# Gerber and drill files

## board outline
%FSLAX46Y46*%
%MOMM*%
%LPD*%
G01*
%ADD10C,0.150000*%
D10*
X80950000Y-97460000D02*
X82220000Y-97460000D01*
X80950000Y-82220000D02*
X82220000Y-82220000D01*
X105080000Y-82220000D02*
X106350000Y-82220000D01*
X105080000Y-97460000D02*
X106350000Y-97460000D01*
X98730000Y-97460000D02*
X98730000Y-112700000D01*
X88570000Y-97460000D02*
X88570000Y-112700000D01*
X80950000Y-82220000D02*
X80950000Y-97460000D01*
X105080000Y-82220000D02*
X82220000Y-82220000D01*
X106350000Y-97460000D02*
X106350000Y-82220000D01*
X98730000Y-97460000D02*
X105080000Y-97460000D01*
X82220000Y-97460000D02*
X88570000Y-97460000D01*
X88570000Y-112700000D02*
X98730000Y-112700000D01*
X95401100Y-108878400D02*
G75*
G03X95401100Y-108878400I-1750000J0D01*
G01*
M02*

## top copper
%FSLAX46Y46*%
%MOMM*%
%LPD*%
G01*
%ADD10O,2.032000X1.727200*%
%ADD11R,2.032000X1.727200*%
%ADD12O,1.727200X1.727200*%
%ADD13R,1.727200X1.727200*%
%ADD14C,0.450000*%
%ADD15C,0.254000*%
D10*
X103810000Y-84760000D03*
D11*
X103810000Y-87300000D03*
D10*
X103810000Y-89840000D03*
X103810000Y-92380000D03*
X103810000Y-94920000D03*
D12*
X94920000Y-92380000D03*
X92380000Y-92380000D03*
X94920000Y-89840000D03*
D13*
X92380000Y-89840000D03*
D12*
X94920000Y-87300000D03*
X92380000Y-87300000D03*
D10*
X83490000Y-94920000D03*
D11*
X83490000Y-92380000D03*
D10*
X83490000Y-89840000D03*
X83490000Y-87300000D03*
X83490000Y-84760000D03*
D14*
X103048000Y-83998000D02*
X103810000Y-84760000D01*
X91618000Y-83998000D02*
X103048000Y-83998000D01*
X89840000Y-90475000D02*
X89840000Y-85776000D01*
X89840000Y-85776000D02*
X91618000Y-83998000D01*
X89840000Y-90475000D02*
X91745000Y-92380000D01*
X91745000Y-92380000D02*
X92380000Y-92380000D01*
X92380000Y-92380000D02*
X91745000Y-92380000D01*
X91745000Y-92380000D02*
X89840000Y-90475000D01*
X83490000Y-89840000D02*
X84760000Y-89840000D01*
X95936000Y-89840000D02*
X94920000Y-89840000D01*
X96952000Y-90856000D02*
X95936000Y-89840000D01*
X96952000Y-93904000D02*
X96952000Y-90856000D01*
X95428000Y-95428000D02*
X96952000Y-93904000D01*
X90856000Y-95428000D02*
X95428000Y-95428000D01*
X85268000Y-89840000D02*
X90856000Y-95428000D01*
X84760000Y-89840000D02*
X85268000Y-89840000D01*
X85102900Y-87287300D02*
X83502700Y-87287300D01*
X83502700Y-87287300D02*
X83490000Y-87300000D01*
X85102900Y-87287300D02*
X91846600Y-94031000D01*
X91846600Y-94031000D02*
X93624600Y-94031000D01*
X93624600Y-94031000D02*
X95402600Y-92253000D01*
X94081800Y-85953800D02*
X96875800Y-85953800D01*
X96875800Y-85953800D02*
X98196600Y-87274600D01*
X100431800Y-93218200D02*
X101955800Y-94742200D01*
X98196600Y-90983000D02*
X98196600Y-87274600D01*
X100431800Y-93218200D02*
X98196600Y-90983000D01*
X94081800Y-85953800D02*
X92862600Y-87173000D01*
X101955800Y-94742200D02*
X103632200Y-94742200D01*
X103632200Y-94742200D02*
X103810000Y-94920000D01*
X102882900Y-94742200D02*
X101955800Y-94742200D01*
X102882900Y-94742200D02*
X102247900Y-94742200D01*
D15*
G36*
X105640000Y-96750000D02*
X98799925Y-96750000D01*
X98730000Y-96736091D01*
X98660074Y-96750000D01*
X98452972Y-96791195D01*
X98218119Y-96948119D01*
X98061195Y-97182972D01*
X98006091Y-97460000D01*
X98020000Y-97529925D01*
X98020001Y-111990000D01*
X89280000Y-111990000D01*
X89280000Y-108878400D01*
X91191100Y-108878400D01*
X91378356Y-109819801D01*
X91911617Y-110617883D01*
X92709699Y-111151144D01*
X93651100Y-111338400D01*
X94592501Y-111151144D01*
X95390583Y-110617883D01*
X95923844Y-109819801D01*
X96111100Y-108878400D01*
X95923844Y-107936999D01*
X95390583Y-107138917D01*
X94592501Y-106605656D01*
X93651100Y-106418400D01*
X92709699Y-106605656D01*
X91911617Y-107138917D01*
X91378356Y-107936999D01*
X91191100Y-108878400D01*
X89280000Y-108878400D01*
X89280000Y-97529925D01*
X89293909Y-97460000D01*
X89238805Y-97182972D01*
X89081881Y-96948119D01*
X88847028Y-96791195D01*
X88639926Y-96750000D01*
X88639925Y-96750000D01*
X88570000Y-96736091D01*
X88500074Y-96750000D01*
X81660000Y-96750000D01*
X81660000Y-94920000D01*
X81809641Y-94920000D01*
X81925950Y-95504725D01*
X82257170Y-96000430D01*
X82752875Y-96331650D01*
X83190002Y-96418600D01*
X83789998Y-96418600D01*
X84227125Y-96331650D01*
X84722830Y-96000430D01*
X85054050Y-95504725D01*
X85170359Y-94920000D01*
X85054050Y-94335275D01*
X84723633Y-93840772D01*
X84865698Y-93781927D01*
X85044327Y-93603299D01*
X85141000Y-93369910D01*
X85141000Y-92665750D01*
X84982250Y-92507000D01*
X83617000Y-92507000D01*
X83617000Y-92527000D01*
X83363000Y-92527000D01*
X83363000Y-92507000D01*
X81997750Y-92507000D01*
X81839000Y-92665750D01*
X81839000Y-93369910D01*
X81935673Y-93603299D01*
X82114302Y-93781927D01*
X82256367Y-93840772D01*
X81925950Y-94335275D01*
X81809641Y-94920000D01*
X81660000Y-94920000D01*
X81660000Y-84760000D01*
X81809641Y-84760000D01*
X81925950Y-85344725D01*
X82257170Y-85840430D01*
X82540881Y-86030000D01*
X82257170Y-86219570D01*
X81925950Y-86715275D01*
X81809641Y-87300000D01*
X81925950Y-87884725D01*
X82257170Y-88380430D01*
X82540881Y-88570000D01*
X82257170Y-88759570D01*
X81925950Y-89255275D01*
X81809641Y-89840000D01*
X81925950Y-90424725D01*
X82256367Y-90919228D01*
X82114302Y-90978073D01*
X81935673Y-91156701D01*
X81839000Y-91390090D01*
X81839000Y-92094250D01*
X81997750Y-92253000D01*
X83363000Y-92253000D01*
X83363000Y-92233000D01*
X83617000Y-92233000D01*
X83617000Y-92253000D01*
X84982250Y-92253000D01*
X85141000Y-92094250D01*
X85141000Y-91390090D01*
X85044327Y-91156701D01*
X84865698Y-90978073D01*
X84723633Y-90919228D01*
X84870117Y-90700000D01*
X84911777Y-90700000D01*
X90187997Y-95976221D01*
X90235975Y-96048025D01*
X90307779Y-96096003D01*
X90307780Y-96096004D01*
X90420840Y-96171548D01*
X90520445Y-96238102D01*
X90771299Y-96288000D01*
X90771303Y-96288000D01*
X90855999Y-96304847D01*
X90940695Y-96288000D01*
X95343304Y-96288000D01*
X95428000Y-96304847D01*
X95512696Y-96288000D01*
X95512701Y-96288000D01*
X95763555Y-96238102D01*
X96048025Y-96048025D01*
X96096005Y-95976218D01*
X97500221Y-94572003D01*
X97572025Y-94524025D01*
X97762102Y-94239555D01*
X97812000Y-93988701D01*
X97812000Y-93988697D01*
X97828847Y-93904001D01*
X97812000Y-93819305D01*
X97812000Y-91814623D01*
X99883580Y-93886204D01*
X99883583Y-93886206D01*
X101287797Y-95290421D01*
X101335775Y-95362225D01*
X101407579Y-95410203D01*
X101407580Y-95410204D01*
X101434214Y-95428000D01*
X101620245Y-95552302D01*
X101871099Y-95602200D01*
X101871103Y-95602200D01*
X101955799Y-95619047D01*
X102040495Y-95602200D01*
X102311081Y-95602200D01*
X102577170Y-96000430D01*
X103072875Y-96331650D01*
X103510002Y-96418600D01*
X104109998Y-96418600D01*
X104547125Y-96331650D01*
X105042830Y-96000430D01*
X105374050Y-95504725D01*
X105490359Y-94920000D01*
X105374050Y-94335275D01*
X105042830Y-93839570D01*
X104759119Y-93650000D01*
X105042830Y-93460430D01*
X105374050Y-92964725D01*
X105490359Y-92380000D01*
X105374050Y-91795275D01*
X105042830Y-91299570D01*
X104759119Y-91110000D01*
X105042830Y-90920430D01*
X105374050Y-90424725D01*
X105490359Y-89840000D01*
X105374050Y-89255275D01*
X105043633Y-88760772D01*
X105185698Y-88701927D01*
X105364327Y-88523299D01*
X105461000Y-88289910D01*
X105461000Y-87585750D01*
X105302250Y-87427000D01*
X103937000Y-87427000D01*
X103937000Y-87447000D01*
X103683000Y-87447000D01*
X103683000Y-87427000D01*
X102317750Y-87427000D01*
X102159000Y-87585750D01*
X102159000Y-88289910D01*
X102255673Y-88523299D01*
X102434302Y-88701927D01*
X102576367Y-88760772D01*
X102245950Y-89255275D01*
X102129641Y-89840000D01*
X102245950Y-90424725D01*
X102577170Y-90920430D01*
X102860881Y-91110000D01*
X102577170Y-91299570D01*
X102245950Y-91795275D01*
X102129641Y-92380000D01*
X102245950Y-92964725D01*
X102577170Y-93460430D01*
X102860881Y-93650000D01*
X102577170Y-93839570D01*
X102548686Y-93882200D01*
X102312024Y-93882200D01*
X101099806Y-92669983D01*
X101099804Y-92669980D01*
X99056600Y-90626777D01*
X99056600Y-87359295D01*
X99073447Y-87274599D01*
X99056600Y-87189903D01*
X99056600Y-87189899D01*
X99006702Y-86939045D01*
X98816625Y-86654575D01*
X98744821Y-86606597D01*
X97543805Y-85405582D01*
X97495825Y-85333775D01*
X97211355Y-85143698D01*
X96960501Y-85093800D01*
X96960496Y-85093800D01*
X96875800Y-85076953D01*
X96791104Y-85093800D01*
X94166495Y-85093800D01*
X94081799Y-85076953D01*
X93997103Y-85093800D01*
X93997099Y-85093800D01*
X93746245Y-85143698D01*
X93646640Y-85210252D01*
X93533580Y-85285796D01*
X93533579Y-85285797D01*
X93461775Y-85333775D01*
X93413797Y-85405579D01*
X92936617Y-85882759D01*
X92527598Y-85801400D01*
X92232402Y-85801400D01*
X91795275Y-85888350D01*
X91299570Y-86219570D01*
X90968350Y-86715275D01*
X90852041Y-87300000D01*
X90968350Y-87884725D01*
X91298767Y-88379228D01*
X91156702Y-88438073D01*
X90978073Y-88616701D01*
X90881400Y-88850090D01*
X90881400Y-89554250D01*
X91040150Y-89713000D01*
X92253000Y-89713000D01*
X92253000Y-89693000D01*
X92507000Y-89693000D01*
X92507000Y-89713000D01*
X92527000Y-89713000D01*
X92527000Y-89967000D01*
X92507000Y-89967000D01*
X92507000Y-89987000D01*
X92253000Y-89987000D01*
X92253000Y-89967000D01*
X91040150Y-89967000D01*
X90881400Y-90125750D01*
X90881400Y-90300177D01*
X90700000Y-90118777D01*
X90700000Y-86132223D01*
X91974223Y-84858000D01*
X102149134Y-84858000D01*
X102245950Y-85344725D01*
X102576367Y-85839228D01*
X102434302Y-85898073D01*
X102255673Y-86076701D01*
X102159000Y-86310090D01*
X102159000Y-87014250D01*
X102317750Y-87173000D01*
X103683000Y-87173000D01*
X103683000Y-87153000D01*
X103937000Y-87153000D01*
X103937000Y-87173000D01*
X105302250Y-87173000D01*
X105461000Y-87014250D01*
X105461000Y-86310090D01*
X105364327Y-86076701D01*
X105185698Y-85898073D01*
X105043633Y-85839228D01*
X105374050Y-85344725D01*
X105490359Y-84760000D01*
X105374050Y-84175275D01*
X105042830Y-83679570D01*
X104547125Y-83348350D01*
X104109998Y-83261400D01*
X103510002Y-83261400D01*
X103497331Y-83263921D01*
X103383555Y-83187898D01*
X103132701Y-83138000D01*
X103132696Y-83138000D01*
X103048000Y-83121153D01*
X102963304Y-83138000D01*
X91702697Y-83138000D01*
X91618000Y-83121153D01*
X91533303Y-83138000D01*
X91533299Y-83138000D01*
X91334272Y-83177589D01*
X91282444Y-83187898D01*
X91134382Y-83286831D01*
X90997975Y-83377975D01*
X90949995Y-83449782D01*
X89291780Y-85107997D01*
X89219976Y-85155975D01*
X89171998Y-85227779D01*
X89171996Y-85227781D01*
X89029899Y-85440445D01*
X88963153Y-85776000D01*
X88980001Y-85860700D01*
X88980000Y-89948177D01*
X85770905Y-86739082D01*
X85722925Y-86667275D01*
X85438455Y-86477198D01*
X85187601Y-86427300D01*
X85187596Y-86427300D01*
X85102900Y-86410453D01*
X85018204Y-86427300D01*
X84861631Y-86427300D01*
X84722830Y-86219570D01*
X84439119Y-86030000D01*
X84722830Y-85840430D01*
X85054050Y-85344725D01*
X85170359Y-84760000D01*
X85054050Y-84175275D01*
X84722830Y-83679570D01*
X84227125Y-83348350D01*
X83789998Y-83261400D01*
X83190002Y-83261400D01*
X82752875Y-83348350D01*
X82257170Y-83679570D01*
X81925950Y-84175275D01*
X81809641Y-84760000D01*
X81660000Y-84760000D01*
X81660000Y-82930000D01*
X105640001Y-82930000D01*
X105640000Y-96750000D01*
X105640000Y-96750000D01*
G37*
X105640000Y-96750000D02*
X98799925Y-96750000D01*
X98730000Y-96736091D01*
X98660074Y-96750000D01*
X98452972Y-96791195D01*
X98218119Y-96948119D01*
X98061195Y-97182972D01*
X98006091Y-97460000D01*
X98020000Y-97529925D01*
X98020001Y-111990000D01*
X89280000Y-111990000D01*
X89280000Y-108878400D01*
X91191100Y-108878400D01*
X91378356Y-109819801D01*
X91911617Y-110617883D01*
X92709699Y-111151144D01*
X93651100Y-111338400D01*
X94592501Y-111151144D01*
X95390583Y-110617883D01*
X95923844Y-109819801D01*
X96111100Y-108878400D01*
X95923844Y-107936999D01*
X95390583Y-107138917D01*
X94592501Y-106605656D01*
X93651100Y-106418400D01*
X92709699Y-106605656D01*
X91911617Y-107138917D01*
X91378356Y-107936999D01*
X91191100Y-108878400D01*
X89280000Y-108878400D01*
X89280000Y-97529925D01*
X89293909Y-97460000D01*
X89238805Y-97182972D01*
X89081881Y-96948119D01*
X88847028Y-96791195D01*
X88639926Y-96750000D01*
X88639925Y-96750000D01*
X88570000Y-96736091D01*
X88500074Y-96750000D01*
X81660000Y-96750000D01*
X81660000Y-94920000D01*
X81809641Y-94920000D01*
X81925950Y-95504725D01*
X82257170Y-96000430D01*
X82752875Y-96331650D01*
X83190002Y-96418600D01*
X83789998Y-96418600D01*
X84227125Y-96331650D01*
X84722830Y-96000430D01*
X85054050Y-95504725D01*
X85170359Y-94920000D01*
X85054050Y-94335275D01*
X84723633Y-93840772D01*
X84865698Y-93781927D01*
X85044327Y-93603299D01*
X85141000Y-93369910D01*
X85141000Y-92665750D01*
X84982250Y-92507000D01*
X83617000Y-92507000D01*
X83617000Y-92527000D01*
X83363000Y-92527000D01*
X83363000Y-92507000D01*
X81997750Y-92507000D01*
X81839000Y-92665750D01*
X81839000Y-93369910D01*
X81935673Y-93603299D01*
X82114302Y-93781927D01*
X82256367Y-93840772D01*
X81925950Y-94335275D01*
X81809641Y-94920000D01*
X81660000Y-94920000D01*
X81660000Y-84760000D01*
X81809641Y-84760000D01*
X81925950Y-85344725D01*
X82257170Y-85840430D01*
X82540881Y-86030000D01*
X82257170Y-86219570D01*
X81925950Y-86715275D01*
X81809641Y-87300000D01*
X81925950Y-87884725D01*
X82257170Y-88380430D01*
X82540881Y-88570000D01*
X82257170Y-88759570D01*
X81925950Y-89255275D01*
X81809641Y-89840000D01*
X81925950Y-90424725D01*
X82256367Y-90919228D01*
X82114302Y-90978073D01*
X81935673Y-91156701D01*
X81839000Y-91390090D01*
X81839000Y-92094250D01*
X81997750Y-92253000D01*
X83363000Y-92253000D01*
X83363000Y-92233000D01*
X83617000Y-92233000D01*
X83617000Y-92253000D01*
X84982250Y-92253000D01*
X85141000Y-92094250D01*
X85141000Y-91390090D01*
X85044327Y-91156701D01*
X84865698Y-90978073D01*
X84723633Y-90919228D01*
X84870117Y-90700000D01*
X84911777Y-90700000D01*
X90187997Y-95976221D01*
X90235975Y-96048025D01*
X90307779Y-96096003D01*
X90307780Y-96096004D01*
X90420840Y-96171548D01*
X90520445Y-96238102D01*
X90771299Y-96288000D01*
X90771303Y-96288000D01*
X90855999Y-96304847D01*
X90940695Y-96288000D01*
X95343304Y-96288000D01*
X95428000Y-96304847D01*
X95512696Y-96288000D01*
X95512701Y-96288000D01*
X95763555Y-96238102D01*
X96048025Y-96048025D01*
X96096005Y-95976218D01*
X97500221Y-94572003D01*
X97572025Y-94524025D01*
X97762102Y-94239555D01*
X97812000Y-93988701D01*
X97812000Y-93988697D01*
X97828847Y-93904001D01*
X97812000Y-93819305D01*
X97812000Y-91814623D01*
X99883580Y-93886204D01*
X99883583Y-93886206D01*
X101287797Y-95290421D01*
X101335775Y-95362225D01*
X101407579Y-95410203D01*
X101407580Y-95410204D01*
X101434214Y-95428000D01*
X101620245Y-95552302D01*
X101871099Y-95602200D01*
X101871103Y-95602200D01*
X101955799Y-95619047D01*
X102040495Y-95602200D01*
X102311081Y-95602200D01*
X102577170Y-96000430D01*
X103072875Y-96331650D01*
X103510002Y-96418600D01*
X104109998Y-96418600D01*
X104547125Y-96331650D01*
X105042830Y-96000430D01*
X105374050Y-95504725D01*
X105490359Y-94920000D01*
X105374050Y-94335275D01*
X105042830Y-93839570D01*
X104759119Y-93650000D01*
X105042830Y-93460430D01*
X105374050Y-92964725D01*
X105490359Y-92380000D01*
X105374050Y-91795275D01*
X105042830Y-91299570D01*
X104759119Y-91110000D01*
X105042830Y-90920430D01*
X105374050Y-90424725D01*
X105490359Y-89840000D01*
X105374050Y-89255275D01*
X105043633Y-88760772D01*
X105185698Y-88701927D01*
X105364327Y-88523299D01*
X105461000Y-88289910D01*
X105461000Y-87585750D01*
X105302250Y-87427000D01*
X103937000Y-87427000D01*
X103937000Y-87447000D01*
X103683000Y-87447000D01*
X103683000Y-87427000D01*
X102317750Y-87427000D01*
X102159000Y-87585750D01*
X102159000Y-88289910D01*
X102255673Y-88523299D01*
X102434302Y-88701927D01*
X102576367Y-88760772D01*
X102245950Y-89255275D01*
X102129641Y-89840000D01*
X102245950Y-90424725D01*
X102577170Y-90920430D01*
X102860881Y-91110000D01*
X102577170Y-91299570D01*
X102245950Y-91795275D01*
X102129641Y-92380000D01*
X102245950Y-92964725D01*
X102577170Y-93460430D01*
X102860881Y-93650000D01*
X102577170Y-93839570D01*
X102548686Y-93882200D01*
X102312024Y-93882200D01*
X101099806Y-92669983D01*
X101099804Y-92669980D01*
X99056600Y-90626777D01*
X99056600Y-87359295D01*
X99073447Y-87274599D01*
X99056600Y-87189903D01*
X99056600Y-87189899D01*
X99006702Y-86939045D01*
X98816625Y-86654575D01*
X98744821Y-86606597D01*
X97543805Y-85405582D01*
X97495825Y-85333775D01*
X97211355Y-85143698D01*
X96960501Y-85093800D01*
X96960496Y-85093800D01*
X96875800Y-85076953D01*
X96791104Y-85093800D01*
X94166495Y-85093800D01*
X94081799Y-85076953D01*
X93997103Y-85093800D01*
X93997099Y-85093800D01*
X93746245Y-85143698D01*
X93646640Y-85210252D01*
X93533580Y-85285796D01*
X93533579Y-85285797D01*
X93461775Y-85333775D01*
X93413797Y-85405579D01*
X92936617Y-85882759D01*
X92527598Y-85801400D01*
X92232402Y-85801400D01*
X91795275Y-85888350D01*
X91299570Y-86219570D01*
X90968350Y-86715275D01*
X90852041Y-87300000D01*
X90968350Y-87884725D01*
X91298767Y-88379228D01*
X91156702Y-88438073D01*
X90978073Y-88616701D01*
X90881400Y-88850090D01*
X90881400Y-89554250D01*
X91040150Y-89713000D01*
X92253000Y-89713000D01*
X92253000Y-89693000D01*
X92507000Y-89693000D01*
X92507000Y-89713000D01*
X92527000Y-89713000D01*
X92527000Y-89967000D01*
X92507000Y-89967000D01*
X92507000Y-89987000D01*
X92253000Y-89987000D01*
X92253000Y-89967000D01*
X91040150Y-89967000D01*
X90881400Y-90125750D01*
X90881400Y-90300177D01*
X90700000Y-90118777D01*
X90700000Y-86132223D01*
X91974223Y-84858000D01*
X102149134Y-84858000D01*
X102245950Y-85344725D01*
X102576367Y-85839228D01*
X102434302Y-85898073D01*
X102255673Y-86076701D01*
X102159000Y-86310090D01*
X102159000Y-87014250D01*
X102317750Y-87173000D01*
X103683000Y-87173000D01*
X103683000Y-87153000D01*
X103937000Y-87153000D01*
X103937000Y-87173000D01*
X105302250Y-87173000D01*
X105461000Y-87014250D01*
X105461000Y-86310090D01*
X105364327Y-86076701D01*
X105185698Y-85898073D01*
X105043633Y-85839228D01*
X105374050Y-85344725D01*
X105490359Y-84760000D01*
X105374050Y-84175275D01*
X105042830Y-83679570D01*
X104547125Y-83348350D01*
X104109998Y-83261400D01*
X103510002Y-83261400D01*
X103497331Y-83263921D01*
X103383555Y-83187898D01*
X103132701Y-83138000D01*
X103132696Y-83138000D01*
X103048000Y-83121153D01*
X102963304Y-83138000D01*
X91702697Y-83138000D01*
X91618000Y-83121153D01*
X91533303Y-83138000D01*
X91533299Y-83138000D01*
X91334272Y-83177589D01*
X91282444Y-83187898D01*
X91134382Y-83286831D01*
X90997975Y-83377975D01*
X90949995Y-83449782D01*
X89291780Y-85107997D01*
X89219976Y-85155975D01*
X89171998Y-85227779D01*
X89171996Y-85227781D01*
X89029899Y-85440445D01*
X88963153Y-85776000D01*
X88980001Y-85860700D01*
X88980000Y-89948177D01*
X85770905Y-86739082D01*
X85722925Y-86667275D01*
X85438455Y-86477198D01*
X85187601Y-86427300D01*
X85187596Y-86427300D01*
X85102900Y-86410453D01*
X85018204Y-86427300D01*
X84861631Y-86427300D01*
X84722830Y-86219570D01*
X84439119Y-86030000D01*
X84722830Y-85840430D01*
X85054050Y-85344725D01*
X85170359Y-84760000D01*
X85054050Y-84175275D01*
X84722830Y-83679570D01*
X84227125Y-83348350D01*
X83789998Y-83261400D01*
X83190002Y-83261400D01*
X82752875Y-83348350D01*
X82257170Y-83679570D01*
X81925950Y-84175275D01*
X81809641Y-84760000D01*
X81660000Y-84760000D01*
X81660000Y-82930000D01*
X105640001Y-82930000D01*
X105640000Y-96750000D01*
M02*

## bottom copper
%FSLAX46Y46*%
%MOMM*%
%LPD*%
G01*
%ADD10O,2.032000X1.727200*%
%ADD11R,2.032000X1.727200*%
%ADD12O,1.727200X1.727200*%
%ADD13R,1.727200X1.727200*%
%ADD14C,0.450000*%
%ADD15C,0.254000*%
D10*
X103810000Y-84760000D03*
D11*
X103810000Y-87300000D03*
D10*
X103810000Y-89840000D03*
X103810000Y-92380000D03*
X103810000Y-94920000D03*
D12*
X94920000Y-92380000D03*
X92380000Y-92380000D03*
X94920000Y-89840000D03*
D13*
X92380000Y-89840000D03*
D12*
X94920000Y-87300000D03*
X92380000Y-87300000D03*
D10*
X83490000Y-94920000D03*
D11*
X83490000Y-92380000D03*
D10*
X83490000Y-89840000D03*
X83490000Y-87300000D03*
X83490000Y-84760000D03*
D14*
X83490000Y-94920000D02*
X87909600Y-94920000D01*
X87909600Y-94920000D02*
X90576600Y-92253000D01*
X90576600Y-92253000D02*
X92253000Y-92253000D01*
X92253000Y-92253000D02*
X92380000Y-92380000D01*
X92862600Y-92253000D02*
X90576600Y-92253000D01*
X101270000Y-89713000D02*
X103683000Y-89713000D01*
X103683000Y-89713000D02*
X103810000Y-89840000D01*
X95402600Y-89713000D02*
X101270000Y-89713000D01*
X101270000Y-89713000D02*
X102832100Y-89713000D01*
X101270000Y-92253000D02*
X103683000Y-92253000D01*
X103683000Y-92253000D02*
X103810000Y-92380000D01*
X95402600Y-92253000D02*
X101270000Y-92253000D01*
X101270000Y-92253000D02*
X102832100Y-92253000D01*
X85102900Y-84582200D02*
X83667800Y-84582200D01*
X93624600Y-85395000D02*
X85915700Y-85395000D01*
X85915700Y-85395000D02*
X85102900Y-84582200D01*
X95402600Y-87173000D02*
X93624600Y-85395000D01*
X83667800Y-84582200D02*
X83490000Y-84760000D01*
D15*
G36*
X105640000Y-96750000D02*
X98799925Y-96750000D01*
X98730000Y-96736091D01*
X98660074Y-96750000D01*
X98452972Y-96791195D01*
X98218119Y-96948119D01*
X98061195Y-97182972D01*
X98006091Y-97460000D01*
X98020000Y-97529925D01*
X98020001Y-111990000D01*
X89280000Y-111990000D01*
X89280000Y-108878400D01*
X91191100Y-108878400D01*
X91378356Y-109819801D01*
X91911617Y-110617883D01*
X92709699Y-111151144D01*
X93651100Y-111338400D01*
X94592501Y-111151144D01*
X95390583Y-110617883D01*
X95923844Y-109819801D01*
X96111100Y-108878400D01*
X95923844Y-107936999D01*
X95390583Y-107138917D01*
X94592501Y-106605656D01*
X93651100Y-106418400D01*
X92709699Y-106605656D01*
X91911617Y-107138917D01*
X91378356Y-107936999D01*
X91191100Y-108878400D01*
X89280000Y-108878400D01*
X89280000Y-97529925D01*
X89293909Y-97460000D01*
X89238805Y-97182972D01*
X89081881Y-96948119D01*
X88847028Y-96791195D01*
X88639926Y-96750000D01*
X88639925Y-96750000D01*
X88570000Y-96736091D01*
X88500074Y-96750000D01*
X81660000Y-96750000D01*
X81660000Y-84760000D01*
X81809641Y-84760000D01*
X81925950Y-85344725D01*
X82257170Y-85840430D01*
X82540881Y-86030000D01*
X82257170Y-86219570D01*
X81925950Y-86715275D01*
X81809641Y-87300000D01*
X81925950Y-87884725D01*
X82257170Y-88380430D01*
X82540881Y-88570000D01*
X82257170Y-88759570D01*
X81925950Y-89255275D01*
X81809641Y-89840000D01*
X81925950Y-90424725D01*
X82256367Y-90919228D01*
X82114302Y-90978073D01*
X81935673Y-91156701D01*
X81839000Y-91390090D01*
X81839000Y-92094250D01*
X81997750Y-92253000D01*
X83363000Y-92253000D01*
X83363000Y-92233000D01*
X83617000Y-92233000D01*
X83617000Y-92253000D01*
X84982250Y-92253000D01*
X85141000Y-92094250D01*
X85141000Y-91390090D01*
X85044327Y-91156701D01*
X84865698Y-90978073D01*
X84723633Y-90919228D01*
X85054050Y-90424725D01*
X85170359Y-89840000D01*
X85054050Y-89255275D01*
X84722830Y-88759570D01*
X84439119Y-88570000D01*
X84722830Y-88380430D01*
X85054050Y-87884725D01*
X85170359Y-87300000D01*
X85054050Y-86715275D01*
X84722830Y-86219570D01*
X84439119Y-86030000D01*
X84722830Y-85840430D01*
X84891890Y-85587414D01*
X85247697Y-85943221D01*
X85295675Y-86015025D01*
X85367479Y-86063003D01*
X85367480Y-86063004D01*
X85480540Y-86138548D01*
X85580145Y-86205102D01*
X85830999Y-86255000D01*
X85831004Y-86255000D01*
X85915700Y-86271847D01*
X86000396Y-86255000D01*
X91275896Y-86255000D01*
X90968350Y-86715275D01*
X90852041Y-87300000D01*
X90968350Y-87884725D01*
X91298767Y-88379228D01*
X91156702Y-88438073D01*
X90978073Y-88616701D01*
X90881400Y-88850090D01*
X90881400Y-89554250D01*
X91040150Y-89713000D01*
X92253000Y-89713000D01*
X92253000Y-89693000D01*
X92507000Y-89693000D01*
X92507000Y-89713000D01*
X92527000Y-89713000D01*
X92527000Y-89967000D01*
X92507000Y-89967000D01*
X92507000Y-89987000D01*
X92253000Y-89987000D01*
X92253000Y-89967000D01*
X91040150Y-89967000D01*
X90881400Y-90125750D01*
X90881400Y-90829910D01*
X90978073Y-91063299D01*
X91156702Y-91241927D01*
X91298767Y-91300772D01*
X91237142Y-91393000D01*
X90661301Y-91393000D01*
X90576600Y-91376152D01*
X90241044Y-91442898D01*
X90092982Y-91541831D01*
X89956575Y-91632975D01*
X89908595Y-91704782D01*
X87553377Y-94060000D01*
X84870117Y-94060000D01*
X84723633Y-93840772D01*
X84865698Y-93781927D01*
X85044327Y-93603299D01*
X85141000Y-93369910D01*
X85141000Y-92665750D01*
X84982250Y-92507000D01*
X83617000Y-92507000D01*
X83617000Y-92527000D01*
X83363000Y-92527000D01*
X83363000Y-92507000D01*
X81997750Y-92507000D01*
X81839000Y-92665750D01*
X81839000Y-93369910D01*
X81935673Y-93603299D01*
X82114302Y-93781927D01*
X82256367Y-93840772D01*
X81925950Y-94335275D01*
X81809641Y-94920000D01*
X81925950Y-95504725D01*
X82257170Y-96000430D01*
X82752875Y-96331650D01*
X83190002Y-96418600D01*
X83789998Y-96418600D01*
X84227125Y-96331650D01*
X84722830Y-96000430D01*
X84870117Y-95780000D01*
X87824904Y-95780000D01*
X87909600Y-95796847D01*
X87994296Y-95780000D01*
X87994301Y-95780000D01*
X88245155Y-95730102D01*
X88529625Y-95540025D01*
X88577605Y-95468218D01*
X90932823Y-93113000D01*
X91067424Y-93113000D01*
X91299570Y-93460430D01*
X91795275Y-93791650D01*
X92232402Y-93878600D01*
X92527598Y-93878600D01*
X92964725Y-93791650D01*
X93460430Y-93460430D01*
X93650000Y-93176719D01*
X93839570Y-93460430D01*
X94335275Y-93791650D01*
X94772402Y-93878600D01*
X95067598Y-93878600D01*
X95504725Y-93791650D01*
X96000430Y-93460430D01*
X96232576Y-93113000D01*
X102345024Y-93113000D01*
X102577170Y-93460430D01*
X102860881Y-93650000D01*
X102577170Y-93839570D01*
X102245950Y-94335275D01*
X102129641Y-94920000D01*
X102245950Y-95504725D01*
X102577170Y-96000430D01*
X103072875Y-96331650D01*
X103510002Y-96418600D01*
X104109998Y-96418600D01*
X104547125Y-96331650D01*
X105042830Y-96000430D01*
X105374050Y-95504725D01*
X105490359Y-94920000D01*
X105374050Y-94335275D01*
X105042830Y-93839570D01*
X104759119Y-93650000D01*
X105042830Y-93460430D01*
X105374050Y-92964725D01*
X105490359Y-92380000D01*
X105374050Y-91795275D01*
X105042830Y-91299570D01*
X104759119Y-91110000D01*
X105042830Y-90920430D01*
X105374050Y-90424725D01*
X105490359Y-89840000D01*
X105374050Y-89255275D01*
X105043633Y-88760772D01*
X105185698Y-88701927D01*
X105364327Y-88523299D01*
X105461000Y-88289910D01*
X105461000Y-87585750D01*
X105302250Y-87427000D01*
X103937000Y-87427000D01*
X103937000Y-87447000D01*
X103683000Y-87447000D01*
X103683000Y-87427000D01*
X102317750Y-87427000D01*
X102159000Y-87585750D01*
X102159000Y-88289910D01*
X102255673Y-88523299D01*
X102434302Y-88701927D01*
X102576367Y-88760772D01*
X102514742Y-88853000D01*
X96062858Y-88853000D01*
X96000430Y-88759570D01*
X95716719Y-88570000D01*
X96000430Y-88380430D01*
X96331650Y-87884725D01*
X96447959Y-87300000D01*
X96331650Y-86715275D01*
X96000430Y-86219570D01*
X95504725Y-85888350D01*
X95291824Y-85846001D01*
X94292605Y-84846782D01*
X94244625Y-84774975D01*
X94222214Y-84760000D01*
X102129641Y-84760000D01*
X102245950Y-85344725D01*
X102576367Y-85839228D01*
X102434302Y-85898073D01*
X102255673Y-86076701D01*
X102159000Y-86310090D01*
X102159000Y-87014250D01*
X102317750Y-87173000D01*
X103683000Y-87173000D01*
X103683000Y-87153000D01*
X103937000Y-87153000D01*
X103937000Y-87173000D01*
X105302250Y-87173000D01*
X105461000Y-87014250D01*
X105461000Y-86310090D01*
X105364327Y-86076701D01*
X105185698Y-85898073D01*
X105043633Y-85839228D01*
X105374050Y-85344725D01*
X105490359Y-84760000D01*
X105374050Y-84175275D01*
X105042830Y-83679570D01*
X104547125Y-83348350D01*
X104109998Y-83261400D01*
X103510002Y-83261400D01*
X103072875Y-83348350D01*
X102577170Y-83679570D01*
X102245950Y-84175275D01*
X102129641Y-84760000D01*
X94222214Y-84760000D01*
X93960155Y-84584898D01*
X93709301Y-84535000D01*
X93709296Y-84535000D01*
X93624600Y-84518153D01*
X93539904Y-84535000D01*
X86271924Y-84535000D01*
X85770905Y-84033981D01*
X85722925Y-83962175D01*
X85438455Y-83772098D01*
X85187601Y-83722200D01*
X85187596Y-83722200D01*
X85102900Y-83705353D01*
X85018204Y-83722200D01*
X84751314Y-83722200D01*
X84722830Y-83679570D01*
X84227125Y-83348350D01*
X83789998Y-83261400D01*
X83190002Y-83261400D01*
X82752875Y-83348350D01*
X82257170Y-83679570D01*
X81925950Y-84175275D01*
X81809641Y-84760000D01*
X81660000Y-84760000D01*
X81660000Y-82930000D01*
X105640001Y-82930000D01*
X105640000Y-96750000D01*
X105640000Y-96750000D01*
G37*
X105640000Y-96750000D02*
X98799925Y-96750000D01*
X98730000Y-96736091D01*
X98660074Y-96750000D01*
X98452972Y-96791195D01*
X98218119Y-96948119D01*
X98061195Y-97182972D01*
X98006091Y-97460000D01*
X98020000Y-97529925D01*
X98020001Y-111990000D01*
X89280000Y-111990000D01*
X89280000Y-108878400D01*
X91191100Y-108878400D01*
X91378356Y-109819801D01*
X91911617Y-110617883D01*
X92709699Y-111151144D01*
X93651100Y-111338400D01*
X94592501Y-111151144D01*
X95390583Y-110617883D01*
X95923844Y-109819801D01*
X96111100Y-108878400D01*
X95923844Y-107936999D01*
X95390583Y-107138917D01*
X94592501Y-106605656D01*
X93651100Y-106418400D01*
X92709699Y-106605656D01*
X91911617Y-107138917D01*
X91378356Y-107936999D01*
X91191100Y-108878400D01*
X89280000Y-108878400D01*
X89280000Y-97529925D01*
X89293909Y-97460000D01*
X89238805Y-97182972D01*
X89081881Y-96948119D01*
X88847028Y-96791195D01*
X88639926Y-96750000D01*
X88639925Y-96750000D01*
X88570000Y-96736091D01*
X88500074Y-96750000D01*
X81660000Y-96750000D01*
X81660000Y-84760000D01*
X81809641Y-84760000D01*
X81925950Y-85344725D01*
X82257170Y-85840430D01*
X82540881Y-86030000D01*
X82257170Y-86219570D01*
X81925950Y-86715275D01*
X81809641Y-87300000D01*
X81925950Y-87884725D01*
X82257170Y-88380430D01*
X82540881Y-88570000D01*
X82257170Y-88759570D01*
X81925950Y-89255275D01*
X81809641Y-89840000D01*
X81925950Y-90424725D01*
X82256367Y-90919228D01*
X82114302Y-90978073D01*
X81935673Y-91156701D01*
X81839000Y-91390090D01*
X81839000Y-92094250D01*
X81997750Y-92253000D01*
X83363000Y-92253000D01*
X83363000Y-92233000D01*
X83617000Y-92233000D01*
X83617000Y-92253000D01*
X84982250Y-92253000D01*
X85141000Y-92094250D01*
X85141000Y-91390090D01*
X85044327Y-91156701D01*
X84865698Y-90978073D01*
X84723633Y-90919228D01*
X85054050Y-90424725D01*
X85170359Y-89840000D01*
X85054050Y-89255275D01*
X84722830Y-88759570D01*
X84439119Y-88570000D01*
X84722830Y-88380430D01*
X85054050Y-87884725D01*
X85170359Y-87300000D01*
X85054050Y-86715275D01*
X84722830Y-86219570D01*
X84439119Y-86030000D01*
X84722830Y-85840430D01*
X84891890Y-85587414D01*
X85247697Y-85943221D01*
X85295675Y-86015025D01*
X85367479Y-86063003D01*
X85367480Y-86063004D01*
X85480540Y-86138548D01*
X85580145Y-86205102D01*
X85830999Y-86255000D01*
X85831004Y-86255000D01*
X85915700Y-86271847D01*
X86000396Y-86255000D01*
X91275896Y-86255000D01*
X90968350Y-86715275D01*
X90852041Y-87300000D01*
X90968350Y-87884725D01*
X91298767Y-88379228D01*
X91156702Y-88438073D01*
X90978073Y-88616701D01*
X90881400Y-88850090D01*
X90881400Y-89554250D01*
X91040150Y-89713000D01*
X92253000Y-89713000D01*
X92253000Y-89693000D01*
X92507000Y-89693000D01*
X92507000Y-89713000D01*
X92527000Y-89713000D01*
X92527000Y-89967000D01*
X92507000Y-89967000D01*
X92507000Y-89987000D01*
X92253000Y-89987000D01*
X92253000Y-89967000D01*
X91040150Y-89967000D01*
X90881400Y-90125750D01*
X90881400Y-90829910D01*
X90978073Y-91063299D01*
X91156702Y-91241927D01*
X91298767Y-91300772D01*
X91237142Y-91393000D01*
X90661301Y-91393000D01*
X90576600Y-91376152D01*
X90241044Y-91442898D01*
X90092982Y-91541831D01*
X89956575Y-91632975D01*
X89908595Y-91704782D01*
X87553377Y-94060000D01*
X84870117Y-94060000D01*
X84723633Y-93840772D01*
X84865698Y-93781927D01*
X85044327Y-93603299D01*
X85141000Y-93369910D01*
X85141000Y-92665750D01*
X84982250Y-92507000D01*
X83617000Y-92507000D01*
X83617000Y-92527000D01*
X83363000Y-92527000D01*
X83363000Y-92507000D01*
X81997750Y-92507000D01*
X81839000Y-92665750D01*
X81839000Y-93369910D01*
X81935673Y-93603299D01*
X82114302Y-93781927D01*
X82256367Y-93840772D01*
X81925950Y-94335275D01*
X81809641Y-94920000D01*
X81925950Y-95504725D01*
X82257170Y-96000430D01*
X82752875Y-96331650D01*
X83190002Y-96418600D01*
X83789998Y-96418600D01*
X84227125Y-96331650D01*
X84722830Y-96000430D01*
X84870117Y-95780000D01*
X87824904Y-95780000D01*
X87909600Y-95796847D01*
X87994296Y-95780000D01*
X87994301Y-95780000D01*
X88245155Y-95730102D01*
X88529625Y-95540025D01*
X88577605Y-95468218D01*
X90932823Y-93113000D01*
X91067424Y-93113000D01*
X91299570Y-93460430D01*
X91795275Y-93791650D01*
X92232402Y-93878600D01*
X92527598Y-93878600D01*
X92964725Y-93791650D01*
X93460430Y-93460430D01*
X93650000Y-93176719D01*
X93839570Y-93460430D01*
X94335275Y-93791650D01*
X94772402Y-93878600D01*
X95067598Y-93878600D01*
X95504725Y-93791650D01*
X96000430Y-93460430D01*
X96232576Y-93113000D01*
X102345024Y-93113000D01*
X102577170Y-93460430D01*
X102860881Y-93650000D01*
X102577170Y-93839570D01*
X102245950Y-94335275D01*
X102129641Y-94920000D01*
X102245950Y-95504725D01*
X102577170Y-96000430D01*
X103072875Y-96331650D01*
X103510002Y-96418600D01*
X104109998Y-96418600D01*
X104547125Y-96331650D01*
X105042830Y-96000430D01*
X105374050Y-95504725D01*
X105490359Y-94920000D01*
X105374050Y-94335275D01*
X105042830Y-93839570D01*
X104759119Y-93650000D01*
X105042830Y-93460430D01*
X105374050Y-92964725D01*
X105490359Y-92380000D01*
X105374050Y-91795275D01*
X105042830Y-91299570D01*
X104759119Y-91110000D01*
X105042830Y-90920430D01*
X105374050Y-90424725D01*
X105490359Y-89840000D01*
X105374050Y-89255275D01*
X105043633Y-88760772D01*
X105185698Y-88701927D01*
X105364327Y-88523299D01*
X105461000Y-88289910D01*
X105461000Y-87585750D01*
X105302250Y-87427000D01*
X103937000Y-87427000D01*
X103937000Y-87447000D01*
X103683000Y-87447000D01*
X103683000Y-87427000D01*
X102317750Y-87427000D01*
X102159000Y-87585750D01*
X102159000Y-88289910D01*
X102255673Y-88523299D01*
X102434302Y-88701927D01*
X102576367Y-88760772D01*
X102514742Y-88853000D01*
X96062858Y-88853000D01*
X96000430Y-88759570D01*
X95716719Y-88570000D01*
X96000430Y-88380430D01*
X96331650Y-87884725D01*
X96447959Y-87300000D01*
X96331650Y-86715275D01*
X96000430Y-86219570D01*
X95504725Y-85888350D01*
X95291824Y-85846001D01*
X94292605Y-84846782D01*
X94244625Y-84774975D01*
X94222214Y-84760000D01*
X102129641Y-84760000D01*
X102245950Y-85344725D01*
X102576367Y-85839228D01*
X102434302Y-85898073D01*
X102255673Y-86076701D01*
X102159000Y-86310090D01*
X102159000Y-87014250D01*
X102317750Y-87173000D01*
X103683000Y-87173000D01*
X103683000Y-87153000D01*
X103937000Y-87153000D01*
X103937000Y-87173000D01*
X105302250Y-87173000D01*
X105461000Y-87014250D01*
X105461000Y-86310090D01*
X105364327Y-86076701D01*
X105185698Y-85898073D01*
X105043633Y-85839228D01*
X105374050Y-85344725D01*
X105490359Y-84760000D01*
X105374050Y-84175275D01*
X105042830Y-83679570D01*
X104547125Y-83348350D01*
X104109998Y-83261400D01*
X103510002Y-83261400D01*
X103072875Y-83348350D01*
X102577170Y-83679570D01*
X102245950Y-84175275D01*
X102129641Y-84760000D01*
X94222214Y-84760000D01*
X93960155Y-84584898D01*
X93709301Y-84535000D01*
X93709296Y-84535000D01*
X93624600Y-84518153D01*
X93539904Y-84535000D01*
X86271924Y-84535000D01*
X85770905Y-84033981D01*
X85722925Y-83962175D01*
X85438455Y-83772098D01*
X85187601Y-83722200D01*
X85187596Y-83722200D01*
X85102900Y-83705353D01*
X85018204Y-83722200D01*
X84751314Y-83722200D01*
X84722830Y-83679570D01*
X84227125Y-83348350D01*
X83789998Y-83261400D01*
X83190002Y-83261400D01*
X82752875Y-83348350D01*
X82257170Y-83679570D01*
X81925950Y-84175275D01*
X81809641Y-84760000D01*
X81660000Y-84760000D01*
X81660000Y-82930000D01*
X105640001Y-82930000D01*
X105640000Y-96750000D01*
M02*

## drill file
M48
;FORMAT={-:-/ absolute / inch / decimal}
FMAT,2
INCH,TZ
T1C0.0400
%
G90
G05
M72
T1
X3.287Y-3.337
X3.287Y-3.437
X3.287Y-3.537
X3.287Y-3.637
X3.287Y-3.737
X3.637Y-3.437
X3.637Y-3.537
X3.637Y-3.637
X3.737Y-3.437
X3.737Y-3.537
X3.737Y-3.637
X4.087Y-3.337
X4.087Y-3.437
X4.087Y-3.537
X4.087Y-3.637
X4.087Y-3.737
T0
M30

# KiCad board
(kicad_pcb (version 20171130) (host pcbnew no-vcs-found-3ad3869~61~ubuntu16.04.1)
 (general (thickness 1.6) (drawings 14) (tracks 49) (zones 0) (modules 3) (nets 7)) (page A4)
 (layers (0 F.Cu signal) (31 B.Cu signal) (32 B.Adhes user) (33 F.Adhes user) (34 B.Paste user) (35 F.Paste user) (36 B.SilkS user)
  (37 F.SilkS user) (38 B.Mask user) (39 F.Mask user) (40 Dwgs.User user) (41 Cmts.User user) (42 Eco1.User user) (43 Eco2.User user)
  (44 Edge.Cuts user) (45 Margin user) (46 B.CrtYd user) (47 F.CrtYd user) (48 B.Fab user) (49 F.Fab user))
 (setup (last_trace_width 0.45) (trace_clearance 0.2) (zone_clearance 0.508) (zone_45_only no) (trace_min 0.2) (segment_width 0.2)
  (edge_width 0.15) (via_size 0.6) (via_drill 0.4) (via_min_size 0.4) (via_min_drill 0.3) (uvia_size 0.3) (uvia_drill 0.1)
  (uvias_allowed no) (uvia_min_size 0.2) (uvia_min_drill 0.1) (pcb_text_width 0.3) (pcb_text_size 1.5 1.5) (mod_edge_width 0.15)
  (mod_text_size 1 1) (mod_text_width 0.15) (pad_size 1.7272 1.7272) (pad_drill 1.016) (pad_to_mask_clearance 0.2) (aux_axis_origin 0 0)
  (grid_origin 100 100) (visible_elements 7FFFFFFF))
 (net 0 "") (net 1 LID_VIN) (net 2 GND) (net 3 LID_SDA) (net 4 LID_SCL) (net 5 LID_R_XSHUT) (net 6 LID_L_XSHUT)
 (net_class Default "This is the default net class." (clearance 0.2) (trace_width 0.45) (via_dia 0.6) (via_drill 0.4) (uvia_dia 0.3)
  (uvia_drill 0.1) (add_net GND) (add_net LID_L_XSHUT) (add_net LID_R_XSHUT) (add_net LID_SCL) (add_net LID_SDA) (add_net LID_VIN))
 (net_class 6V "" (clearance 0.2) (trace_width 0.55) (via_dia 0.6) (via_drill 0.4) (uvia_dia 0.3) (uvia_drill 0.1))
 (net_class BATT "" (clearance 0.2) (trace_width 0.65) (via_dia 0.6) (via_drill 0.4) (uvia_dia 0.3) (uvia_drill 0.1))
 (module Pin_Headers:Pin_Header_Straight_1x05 (layer F.Cu) (at 103.81 84.76)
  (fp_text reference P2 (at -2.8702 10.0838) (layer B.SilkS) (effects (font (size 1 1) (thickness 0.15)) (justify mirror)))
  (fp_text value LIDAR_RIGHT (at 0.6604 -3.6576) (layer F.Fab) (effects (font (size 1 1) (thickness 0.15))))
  (pad 1 thru_hole oval (at 0 0) (size 2.032 1.7272) (drill 1.016) (layers *.Cu *.Mask F.SilkS) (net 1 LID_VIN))
  (pad 2 thru_hole rect (at 0 2.54) (size 2.032 1.7272) (drill 1.016) (layers *.Cu *.Mask F.SilkS) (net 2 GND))
  (pad 3 thru_hole oval (at 0 5.08) (size 2.032 1.7272) (drill 1.016) (layers *.Cu *.Mask F.SilkS) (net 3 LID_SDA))
  (pad 4 thru_hole oval (at 0 7.62) (size 2.032 1.7272) (drill 1.016) (layers *.Cu *.Mask F.SilkS) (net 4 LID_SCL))
  (pad 5 thru_hole oval (at 0 10.16) (size 2.032 1.7272) (drill 1.016) (layers *.Cu *.Mask F.SilkS) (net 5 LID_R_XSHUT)))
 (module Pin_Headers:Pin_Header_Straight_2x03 (layer F.Cu) (at 94.92 92.38 180)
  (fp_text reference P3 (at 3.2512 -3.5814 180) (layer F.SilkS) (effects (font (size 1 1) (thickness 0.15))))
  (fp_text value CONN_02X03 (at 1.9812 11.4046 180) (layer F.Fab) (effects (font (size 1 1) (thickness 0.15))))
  (pad 1 thru_hole oval (at 0 0 180) (size 1.7272 1.7272) (drill 1.016) (layers *.Cu *.Mask F.SilkS) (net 4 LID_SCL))
  (pad 2 thru_hole oval (at 2.54 0 180) (size 1.7272 1.7272) (drill 1.016) (layers *.Cu *.Mask F.SilkS) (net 1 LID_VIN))
  (pad 3 thru_hole oval (at 0 2.54 180) (size 1.7272 1.7272) (drill 1.016) (layers *.Cu *.Mask F.SilkS) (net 3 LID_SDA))
  (pad 4 thru_hole rect (at 2.54 2.54 180) (size 1.7272 1.7272) (drill 1.016) (layers *.Cu *.Mask F.SilkS) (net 2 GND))
  (pad 5 thru_hole oval (at 0 5.08 180) (size 1.7272 1.7272) (drill 1.016) (layers *.Cu *.Mask F.SilkS) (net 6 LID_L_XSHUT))
  (pad 6 thru_hole oval (at 2.54 5.08 180) (size 1.7272 1.7272) (drill 1.016) (layers *.Cu *.Mask F.SilkS) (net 5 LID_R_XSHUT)))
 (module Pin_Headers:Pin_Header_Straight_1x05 (layer F.Cu) (at 83.49 94.92 180)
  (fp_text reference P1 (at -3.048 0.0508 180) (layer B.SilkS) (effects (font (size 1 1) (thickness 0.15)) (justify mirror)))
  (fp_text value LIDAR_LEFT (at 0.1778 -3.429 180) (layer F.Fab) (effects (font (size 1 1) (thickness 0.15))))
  (pad 1 thru_hole oval (at 0 0 180) (size 2.032 1.7272) (drill 1.016) (layers *.Cu *.Mask F.SilkS) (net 1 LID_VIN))
  (pad 2 thru_hole rect (at 0 2.54 180) (size 2.032 1.7272) (drill 1.016) (layers *.Cu *.Mask F.SilkS) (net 2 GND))
  (pad 3 thru_hole oval (at 0 5.08 180) (size 2.032 1.7272) (drill 1.016) (layers *.Cu *.Mask F.SilkS) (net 3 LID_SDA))
  (pad 4 thru_hole oval (at 0 7.62 180) (size 2.032 1.7272) (drill 1.016) (layers *.Cu *.Mask F.SilkS) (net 4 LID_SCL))
  (pad 5 thru_hole oval (at 0 10.16 180) (size 2.032 1.7272) (drill 1.016) (layers *.Cu *.Mask F.SilkS) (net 6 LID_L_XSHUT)))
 (gr_line (start 80.95 97.46) (end 82.22 97.46) (angle 90) (layer Edge.Cuts) (width 0.15))
 (gr_line (start 80.95 82.22) (end 82.22 82.22) (angle 90) (layer Edge.Cuts) (width 0.15))
 (gr_line (start 105.08 82.22) (end 106.35 82.22) (angle 90) (layer Edge.Cuts) (width 0.15))
 (gr_line (start 105.08 97.46) (end 106.35 97.46) (angle 90) (layer Edge.Cuts) (width 0.15))
 (gr_line (start 98.73 97.46) (end 98.73 112.7) (angle 90) (layer Edge.Cuts) (width 0.15))
 (gr_line (start 88.57 97.46) (end 88.57 112.7) (angle 90) (layer Edge.Cuts) (width 0.15))
 (gr_line (start 80.95 82.22) (end 80.95 97.46) (angle 90) (layer Edge.Cuts) (width 0.15))
 (gr_line (start 105.08 82.22) (end 82.22 82.22) (angle 90) (layer Edge.Cuts) (width 0.15))
 (gr_line (start 106.35 97.46) (end 106.35 82.22) (angle 90) (layer Edge.Cuts) (width 0.15))
 (gr_line (start 98.73 97.46) (end 105.08 97.46) (angle 90) (layer Edge.Cuts) (width 0.15))
 (gr_line (start 82.22 97.46) (end 88.57 97.46) (angle 90) (layer Edge.Cuts) (width 0.15))
 (gr_line (start 88.57 112.7) (end 98.73 112.7) (angle 90) (layer Edge.Cuts) (width 0.15))
 (gr_circle (center 93.6511 108.8784) (end 95.4011 108.8784) (layer Edge.Cuts) (width 0.15))
 (segment (start 103.048 83.998) (end 103.81 84.76) (width 0.45) (layer F.Cu) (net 1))
 (segment (start 91.618 83.998) (end 103.048 83.998) (width 0.45) (layer F.Cu) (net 1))
 (segment (start 89.84 90.475) (end 89.84 85.776) (width 0.45) (layer F.Cu) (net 1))
 (segment (start 89.84 85.776) (end 91.618 83.998) (width 0.45) (layer F.Cu) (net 1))
 (segment (start 83.49 94.92) (end 87.9096 94.92) (width 0.45) (layer B.Cu) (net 1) (status 400000))
 (segment (start 87.9096 94.92) (end 90.5766 92.253) (width 0.45) (layer B.Cu) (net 1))
 (segment (start 90.5766 92.253) (end 92.253 92.253) (width 0.45) (layer B.Cu) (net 1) (status 800000))
 (segment (start 92.253 92.253) (end 92.38 92.38) (width 0.45) (layer B.Cu) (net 1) (status C00000))
 (segment (start 89.84 90.475) (end 91.745 92.38) (width 0.45) (layer F.Cu) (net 1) (status 800000))
 (segment (start 91.745 92.38) (end 92.38 92.38) (width 0.45) (layer F.Cu) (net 1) (status C00000))
 (segment (start 92.38 92.38) (end 91.745 92.38) (width 0.45) (layer F.Cu) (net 1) (status C00000))
 (segment (start 91.745 92.38) (end 89.84 90.475) (width 0.45) (layer F.Cu) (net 1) (status 400000))
 (segment (start 92.8626 92.253) (end 90.5766 92.253) (width 0.45) (layer B.Cu) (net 1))
 (segment (start 101.27 89.713) (end 103.683 89.713) (width 0.45) (layer B.Cu) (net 3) (status 800000))
 (segment (start 103.683 89.713) (end 103.81 89.84) (width 0.45) (layer B.Cu) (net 3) (status C00000))
 (segment (start 83.49 89.84) (end 84.76 89.84) (width 0.45) (layer F.Cu) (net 3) (status 400000))
 (segment (start 95.936 89.84) (end 94.92 89.84) (width 0.45) (layer F.Cu) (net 3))
 (segment (start 96.952 90.856) (end 95.936 89.84) (width 0.45) (layer F.Cu) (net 3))
 (segment (start 96.952 93.904) (end 96.952 90.856) (width 0.45) (layer F.Cu) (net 3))
 (segment (start 95.428 95.428) (end 96.952 93.904) (width 0.45) (layer F.Cu) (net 3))
 (segment (start 90.856 95.428) (end 95.428 95.428) (width 0.45) (layer F.Cu) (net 3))
 (segment (start 85.268 89.84) (end 90.856 95.428) (width 0.45) (layer F.Cu) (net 3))
 (segment (start 84.76 89.84) (end 85.268 89.84) (width 0.45) (layer F.Cu) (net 3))
 (segment (start 95.4026 89.713) (end 101.27 89.713) (width 0.45) (layer B.Cu) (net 3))
 (segment (start 101.27 89.713) (end 102.8321 89.713) (width 0.45) (layer B.Cu) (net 3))
 (segment (start 101.27 92.253) (end 103.683 92.253) (width 0.45) (layer B.Cu) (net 4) (status 800000))
 (segment (start 103.683 92.253) (end 103.81 92.38) (width 0.45) (layer B.Cu) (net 4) (status C00000))
 (segment (start 85.1029 87.2873) (end 83.5027 87.2873) (width 0.45) (layer F.Cu) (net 4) (status 800000))
 (segment (start 83.5027 87.2873) (end 83.49 87.3) (width 0.45) (layer F.Cu) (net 4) (status C00000))
 (segment (start 85.1029 87.2873) (end 91.8466 94.031) (width 0.45) (layer F.Cu) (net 4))
 (segment (start 91.8466 94.031) (end 93.6246 94.031) (width 0.45) (layer F.Cu) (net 4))
 (segment (start 93.6246 94.031) (end 95.4026 92.253) (width 0.45) (layer F.Cu) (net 4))
 (segment (start 95.4026 92.253) (end 101.27 92.253) (width 0.45) (layer B.Cu) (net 4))
 (segment (start 101.27 92.253) (end 102.8321 92.253) (width 0.45) (layer B.Cu) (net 4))
 (segment (start 85.1029 84.5822) (end 83.6678 84.5822) (width 0.45) (layer B.Cu) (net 6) (status 800000))
 (segment (start 93.6246 85.395) (end 85.9157 85.395) (width 0.45) (layer B.Cu) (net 6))
 (segment (start 85.9157 85.395) (end 85.1029 84.5822) (width 0.45) (layer B.Cu) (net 6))
 (segment (start 95.4026 87.173) (end 93.6246 85.395) (width 0.45) (layer B.Cu) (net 6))
 (segment (start 83.6678 84.5822) (end 83.49 84.76) (width 0.45) (layer B.Cu) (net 6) (status C00000))
 (segment (start 94.0818 85.9538) (end 96.8758 85.9538) (width 0.45) (layer F.Cu) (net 5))
 (segment (start 96.8758 85.9538) (end 98.1966 87.2746) (width 0.45) (layer F.Cu) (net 5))
 (segment (start 100.4318 93.2182) (end 101.9558 94.7422) (width 0.45) (layer F.Cu) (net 5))
 (segment (start 98.1966 90.983) (end 98.1966 87.2746) (width 0.45) (layer F.Cu) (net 5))
 (segment (start 100.4318 93.2182) (end 98.1966 90.983) (width 0.45) (layer F.Cu) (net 5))
 (segment (start 94.0818 85.9538) (end 92.8626 87.173) (width 0.45) (layer F.Cu) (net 5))
 (segment (start 101.9558 94.7422) (end 103.6322 94.7422) (width 0.45) (layer F.Cu) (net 5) (status 800000))
 (segment (start 103.6322 94.7422) (end 103.81 94.92) (width 0.45) (layer F.Cu) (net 5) (status C00000))
 (segment (start 102.8829 94.7422) (end 101.9558 94.7422) (width 0.45) (layer F.Cu) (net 5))
 (segment (start 102.8829 94.7422) (end 102.2479 94.7422) (width 0.45) (layer F.Cu) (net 5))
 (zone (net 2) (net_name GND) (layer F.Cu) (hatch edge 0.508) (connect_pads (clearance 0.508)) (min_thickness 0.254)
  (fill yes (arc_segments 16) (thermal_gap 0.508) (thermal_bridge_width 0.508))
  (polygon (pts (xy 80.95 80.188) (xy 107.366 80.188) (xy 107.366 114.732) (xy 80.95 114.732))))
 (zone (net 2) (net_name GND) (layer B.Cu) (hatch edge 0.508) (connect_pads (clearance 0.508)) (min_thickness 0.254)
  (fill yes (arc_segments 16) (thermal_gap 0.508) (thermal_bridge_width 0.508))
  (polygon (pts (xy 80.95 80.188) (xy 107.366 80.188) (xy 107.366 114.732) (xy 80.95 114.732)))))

